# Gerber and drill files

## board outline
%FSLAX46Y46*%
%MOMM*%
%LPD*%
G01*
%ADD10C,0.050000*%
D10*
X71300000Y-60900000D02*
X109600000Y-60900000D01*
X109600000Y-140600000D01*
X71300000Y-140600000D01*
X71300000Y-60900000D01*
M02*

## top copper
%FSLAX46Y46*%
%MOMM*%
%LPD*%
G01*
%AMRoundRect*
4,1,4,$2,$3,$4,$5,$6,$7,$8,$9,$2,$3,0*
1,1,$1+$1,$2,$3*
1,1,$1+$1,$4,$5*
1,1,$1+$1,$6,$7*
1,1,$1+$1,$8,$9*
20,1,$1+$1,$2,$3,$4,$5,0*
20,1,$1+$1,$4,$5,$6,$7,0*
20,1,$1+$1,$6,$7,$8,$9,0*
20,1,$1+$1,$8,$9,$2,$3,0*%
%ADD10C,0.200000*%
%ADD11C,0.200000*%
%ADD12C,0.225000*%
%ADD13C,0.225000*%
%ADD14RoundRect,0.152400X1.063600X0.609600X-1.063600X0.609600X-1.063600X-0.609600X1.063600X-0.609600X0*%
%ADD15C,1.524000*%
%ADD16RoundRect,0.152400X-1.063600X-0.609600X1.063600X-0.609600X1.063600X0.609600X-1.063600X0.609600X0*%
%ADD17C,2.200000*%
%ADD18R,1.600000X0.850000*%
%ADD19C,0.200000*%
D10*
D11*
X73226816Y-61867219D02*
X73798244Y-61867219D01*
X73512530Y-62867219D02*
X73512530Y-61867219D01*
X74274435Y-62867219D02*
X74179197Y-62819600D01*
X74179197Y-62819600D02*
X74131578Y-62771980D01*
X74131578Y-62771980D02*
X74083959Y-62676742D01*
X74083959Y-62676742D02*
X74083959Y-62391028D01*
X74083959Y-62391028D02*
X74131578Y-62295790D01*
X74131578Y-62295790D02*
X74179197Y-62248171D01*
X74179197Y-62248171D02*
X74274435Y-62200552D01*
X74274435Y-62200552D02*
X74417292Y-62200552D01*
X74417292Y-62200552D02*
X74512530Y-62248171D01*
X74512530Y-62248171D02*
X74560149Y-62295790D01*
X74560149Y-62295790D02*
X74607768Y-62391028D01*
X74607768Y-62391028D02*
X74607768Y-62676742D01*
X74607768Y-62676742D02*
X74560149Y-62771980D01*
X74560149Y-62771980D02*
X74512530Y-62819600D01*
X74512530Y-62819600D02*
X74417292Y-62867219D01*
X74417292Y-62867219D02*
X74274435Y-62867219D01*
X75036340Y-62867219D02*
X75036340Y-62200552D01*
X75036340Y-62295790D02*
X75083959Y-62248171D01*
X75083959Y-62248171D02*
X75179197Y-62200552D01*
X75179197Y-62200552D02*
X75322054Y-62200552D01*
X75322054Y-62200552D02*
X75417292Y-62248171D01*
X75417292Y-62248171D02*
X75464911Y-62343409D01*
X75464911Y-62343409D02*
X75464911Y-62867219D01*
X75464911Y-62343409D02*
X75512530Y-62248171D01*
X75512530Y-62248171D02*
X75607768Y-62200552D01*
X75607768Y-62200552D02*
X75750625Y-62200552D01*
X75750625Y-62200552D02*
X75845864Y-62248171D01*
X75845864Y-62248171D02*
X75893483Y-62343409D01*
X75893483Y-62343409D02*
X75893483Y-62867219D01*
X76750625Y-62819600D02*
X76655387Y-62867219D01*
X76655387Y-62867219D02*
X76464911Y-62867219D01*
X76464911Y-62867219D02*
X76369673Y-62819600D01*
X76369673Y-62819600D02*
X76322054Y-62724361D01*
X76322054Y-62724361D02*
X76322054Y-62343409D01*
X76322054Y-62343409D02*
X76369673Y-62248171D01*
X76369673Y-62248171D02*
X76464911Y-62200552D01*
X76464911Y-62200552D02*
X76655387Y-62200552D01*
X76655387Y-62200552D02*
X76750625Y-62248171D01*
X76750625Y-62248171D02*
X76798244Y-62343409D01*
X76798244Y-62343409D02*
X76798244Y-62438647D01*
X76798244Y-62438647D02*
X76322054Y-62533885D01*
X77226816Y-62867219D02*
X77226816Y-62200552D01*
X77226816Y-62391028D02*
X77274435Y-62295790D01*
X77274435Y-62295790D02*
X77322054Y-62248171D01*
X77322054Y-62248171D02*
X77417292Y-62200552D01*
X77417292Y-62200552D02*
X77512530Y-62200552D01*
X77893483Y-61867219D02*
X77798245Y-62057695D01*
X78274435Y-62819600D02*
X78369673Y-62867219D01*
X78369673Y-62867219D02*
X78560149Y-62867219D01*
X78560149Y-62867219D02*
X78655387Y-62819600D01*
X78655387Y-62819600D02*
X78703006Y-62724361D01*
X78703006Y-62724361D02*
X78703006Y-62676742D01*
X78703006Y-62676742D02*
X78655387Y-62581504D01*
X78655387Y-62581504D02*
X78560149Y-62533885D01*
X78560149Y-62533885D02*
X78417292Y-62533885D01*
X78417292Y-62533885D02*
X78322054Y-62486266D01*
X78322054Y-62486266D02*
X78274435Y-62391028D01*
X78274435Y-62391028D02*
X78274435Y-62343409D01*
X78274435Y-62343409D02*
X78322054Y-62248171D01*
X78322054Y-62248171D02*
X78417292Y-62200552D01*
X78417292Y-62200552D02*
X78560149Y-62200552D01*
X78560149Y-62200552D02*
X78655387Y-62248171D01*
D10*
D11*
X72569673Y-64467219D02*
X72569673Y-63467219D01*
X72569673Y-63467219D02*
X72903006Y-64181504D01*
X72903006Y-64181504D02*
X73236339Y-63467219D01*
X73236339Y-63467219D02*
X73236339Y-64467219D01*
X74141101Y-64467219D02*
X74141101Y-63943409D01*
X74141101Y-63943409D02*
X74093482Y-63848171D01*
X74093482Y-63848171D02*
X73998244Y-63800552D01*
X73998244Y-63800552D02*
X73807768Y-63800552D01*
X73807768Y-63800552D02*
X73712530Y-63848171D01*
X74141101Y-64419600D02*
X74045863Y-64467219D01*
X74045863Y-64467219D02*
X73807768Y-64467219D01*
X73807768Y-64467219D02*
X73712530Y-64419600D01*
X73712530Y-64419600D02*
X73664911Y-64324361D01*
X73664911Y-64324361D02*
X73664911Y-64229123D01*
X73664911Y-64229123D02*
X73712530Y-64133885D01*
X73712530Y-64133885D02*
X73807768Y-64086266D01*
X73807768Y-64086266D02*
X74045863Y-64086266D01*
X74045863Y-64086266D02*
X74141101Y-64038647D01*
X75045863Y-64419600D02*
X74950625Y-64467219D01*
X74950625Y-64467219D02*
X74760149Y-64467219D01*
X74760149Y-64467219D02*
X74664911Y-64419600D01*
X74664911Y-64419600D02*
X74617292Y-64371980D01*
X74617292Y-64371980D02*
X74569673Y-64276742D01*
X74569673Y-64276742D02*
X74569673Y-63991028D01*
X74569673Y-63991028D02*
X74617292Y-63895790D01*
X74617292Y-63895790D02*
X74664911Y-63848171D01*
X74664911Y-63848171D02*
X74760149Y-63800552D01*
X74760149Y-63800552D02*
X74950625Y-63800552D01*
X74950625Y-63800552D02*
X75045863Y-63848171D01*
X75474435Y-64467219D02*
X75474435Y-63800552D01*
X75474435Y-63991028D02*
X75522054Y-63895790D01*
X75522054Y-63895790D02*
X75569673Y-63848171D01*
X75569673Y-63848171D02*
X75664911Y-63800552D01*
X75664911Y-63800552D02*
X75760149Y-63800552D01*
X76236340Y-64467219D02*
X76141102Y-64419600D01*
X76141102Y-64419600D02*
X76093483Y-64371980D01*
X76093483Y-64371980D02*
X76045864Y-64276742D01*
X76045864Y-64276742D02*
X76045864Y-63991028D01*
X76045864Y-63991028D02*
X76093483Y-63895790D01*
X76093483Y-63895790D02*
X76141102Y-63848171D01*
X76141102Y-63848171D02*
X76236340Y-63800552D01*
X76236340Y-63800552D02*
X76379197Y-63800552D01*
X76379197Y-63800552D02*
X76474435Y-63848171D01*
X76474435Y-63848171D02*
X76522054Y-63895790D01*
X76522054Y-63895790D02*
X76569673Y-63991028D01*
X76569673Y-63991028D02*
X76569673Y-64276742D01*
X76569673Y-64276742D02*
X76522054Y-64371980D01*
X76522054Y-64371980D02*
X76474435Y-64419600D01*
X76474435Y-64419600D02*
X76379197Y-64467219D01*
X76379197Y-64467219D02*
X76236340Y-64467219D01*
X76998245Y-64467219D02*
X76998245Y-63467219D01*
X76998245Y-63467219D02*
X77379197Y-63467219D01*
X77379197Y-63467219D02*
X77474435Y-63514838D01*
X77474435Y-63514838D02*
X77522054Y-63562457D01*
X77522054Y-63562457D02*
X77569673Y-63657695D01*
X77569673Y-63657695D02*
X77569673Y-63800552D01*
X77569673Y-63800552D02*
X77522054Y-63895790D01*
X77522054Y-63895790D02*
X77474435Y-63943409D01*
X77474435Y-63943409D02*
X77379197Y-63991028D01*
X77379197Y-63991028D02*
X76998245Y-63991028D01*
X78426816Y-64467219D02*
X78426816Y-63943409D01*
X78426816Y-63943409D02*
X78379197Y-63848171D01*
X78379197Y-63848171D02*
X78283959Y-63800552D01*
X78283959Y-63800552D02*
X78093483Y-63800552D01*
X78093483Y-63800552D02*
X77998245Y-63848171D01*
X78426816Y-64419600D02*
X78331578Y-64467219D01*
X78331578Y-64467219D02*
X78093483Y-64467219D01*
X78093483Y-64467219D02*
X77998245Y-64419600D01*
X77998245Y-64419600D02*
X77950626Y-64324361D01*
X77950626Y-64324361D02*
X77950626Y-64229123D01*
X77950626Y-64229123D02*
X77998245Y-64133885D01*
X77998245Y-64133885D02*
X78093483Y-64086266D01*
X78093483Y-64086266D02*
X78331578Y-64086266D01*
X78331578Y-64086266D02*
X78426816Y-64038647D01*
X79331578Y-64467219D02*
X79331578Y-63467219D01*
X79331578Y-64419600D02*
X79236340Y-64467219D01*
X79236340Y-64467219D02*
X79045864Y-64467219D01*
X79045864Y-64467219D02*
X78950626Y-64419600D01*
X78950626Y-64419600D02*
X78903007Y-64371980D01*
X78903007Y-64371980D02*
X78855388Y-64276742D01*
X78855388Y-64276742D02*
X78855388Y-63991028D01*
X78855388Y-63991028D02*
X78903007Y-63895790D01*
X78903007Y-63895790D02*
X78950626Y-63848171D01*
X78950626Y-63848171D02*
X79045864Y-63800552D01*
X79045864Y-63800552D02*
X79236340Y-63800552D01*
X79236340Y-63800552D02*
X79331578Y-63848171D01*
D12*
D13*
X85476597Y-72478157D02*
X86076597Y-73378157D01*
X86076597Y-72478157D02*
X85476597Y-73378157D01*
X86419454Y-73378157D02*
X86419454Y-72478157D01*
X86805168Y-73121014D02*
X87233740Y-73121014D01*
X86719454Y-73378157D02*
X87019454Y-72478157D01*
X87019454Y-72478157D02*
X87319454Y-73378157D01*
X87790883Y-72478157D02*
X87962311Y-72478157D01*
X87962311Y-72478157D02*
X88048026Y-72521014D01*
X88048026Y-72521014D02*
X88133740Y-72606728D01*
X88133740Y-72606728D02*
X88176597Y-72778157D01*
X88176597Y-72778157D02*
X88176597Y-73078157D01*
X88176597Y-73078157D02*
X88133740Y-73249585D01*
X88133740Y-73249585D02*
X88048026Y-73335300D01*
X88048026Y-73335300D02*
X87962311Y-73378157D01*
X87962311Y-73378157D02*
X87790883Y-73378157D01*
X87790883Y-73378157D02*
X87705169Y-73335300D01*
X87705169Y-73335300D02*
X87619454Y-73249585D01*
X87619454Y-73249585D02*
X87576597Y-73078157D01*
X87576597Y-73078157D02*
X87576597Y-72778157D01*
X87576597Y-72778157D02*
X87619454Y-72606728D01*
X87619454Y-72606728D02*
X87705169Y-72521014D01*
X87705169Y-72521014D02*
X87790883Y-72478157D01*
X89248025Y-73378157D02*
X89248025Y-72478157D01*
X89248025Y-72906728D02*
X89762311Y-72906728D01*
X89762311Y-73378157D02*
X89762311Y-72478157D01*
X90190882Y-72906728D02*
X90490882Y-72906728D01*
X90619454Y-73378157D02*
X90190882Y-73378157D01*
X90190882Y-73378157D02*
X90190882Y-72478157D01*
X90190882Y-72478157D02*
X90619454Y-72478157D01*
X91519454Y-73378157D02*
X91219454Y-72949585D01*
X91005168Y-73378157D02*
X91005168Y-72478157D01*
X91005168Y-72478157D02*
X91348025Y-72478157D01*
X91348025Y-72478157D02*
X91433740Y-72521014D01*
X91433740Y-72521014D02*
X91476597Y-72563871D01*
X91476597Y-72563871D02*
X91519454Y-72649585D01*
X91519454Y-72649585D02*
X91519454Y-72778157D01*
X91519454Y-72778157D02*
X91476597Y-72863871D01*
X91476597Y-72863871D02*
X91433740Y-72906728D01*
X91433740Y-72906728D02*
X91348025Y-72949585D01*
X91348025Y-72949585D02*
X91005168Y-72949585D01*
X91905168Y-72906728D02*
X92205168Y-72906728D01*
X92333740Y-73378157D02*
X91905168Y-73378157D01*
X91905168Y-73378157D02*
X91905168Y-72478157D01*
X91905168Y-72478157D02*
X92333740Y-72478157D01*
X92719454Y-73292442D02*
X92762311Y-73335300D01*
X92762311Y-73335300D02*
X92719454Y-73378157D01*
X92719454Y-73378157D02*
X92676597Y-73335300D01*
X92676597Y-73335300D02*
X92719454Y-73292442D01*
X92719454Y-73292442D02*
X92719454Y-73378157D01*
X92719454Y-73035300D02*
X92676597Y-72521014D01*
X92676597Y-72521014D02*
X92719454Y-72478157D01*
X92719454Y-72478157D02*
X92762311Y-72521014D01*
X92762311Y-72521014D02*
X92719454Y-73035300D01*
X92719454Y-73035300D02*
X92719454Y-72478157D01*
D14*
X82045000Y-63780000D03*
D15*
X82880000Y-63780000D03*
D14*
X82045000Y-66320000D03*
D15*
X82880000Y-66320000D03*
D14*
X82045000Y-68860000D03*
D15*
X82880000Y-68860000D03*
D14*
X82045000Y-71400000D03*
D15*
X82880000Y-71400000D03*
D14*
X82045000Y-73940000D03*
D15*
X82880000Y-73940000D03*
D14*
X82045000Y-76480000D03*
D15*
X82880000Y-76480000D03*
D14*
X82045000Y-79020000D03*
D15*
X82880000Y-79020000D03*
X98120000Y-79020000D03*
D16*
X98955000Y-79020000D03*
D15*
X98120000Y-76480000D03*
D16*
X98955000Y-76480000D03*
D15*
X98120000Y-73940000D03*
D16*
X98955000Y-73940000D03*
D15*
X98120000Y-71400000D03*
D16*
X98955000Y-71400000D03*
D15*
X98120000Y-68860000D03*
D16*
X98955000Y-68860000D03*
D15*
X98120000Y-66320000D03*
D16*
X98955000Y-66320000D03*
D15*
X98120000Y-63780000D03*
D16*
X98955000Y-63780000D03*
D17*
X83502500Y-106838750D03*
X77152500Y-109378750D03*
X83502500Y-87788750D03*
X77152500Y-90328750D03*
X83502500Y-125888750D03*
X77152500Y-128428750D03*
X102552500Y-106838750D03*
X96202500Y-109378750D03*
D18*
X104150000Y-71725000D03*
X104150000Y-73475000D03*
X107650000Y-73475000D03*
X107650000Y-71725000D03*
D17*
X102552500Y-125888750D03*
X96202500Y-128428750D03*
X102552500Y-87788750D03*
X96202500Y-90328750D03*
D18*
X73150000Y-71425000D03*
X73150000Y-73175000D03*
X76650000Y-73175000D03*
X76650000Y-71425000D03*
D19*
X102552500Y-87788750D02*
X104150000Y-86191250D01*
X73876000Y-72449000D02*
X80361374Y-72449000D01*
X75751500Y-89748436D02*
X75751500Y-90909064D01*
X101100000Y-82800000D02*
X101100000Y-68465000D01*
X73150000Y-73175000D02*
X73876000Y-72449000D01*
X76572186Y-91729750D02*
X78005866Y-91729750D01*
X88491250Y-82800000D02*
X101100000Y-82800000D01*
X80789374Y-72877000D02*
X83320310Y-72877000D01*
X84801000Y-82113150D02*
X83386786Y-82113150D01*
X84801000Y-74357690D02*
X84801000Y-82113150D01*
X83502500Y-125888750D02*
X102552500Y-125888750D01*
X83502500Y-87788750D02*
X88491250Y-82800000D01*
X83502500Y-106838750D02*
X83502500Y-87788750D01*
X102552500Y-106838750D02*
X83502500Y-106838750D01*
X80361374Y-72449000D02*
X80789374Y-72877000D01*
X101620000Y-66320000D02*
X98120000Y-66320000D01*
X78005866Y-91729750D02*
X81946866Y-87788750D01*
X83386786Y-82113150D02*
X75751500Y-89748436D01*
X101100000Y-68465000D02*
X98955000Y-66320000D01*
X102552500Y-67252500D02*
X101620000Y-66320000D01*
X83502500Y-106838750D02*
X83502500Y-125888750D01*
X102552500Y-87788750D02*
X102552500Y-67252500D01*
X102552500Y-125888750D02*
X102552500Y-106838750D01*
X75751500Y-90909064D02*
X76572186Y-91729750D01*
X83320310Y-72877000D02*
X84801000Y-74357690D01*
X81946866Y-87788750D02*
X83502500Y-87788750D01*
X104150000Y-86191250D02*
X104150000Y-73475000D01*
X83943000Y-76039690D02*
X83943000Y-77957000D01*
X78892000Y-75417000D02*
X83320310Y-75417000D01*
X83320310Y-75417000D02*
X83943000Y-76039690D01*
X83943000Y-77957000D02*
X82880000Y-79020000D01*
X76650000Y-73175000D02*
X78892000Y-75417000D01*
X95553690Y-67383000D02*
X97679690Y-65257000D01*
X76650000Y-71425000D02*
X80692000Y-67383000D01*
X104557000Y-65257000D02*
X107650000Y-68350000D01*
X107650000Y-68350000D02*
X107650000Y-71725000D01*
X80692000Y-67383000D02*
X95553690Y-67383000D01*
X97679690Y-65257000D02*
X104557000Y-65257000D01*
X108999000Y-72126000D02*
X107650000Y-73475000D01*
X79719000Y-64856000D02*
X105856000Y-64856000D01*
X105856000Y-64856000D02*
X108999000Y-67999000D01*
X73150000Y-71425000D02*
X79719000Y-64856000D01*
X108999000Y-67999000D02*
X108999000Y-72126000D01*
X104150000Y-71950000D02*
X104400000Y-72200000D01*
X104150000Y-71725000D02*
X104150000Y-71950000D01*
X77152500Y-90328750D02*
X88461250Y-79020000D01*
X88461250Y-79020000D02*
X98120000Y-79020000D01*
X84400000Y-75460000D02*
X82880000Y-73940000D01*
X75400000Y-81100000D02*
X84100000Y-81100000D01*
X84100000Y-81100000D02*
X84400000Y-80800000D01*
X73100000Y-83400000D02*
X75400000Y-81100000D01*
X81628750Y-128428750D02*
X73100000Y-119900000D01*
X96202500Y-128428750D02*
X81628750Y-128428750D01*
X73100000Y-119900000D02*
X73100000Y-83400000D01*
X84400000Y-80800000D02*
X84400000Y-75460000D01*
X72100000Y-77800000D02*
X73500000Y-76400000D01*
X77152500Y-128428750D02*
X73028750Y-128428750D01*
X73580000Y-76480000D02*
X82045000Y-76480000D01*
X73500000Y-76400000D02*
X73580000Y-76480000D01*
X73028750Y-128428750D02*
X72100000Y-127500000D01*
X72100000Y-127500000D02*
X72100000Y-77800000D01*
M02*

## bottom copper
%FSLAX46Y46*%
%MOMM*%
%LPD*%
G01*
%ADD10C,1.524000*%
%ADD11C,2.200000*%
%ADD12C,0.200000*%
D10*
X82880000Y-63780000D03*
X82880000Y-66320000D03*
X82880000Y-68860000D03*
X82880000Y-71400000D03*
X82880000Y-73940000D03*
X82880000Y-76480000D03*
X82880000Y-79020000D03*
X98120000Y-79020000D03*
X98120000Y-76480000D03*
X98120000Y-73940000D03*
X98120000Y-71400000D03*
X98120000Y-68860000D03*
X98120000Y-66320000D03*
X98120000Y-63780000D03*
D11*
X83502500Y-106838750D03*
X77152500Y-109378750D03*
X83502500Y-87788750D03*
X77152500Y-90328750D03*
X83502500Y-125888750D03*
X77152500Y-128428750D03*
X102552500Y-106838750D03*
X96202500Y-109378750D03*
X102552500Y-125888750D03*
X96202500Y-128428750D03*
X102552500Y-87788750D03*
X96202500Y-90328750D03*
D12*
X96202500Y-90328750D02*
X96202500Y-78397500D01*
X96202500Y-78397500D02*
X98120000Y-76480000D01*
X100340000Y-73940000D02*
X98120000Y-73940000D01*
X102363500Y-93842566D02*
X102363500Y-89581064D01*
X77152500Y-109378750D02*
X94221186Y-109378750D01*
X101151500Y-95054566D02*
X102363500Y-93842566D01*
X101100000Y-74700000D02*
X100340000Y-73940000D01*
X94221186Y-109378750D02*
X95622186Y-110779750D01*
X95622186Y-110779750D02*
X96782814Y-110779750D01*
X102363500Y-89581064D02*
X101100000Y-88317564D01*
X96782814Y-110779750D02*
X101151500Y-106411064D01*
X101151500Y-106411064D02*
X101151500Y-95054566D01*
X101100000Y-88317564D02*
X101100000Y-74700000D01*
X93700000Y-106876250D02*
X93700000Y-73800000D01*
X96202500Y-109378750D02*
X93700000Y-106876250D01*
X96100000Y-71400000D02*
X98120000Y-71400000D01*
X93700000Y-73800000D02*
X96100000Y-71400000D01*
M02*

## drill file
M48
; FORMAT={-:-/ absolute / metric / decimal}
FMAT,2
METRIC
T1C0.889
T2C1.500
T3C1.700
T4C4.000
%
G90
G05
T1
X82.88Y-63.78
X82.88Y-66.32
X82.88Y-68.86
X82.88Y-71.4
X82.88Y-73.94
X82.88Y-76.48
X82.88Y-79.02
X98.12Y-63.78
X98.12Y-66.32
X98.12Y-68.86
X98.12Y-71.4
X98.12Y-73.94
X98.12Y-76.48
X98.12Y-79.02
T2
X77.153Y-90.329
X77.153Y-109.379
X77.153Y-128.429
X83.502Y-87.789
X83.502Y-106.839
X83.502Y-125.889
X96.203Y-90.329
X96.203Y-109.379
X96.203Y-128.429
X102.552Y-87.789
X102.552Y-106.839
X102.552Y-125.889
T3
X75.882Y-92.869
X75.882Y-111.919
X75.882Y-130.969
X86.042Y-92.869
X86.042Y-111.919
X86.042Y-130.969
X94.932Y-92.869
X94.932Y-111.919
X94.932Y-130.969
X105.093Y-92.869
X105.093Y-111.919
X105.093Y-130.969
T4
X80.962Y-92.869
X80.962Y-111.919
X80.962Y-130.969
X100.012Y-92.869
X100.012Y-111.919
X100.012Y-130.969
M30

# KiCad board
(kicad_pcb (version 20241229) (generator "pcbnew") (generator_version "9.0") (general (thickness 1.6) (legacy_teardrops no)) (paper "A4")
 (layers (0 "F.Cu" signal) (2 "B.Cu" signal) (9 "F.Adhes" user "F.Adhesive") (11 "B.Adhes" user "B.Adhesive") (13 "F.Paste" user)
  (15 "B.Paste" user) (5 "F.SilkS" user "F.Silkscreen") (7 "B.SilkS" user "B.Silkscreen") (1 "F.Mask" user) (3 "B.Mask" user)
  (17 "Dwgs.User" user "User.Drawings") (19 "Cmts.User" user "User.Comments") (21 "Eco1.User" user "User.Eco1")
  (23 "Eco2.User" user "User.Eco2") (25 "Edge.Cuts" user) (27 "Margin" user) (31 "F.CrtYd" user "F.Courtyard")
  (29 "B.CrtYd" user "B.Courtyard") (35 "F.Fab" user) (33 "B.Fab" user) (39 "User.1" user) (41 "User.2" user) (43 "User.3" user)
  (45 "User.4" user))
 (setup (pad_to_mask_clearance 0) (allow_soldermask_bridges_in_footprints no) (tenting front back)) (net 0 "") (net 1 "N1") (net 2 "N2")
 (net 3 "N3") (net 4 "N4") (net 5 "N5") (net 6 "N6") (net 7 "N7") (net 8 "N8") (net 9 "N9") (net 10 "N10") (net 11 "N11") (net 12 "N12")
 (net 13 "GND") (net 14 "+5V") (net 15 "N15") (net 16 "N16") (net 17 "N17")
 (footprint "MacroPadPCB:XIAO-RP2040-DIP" (layer "F.Cu") (at 90.5 71.4)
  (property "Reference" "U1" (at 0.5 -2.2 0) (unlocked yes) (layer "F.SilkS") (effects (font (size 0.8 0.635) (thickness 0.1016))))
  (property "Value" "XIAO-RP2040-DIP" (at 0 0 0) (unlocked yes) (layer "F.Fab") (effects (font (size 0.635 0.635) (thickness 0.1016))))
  (pad "1" smd roundrect (at -8.455 -7.62 180) (size 2.432 1.524) (layers "F.Cu" "F.Mask") (roundrect_rratio 0.1) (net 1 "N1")
   (thermal_bridge_angle 45))
  (pad "1" thru_hole circle (at -7.62 -7.62 180) (size 1.524 1.524) (drill 0.889) (layers "*.Cu" "*.Mask") (remove_unused_layers no)
   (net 1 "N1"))
  (pad "2" smd roundrect (at -8.455 -5.08 180) (size 2.432 1.524) (layers "F.Cu" "F.Mask") (roundrect_rratio 0.1) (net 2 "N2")
   (thermal_bridge_angle 45))
  (pad "2" thru_hole circle (at -7.62 -5.08 180) (size 1.524 1.524) (drill 0.889) (layers "*.Cu" "*.Mask") (remove_unused_layers no)
   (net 2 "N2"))
  (pad "3" smd roundrect (at -8.455 -2.54 180) (size 2.432 1.524) (layers "F.Cu" "F.Mask") (roundrect_rratio 0.1) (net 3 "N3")
   (thermal_bridge_angle 45))
  (pad "3" thru_hole circle (at -7.62 -2.54 180) (size 1.524 1.524) (drill 0.889) (layers "*.Cu" "*.Mask") (remove_unused_layers no)
   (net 3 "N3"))
  (pad "4" smd roundrect (at -8.455 0 180) (size 2.432 1.524) (layers "F.Cu" "F.Mask") (roundrect_rratio 0.1) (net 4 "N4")
   (thermal_bridge_angle 45))
  (pad "4" thru_hole circle (at -7.62 0 180) (size 1.524 1.524) (drill 0.889) (layers "*.Cu" "*.Mask") (remove_unused_layers no)
   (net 4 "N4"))
  (pad "5" smd roundrect (at -8.455 2.54 180) (size 2.432 1.524) (layers "F.Cu" "F.Mask") (roundrect_rratio 0.1) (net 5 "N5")
   (thermal_bridge_angle 45))
  (pad "5" thru_hole circle (at -7.62 2.54 180) (size 1.524 1.524) (drill 0.889) (layers "*.Cu" "*.Mask") (remove_unused_layers no)
   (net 5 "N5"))
  (pad "6" smd roundrect (at -8.455 5.08 180) (size 2.432 1.524) (layers "F.Cu" "F.Mask") (roundrect_rratio 0.1) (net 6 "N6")
   (thermal_bridge_angle 45))
  (pad "6" thru_hole circle (at -7.62 5.08 180) (size 1.524 1.524) (drill 0.889) (layers "*.Cu" "*.Mask") (remove_unused_layers no)
   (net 6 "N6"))
  (pad "7" smd roundrect (at -8.455 7.62 180) (size 2.432 1.524) (layers "F.Cu" "F.Mask") (roundrect_rratio 0.1) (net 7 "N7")
   (thermal_bridge_angle 45))
  (pad "7" thru_hole circle (at -7.62 7.62 180) (size 1.524 1.524) (drill 0.889) (layers "*.Cu" "*.Mask") (remove_unused_layers no)
   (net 7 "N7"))
  (pad "8" thru_hole circle (at 7.62 7.62) (size 1.524 1.524) (drill 0.889) (layers "*.Cu" "*.Mask") (remove_unused_layers no) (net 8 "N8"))
  (pad "8" smd roundrect (at 8.455 7.62) (size 2.432 1.524) (layers "F.Cu" "F.Mask") (roundrect_rratio 0.1) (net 8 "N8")
   (thermal_bridge_angle 45))
  (pad "9" thru_hole circle (at 7.62 5.08) (size 1.524 1.524) (drill 0.889) (layers "*.Cu" "*.Mask") (remove_unused_layers no) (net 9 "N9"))
  (pad "9" smd roundrect (at 8.455 5.08) (size 2.432 1.524) (layers "F.Cu" "F.Mask") (roundrect_rratio 0.1) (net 9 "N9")
   (thermal_bridge_angle 45))
  (pad "10" thru_hole circle (at 7.62 2.54) (size 1.524 1.524) (drill 0.889) (layers "*.Cu" "*.Mask") (remove_unused_layers no)
   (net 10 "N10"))
  (pad "10" smd roundrect (at 8.455 2.54) (size 2.432 1.524) (layers "F.Cu" "F.Mask") (roundrect_rratio 0.1) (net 10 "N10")
   (thermal_bridge_angle 45))
  (pad "11" thru_hole circle (at 7.62 0) (size 1.524 1.524) (drill 0.889) (layers "*.Cu" "*.Mask") (remove_unused_layers no) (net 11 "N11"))
  (pad "11" smd roundrect (at 8.455 0) (size 2.432 1.524) (layers "F.Cu" "F.Mask") (roundrect_rratio 0.1) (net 11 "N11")
   (thermal_bridge_angle 45))
  (pad "12" thru_hole circle (at 7.62 -2.54) (size 1.524 1.524) (drill 0.889) (layers "*.Cu" "*.Mask") (remove_unused_layers no)
   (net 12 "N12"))
  (pad "12" smd roundrect (at 8.455 -2.54) (size 2.432 1.524) (layers "F.Cu" "F.Mask") (roundrect_rratio 0.1) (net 12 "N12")
   (thermal_bridge_angle 45))
  (pad "13" thru_hole circle (at 7.62 -5.08) (size 1.524 1.524) (drill 0.889) (layers "*.Cu" "*.Mask") (remove_unused_layers no)
   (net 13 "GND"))
  (pad "13" smd roundrect (at 8.455 -5.08) (size 2.432 1.524) (layers "F.Cu" "F.Mask") (roundrect_rratio 0.1) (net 13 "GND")
   (thermal_bridge_angle 45))
  (pad "14" thru_hole circle (at 7.62 -7.62) (size 1.524 1.524) (drill 0.889) (layers "*.Cu" "*.Mask") (remove_unused_layers no)
   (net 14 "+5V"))
  (pad "14" smd roundrect (at 8.455 -7.62) (size 2.432 1.524) (layers "F.Cu" "F.Mask") (roundrect_rratio 0.1) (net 14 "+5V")
   (thermal_bridge_angle 45)))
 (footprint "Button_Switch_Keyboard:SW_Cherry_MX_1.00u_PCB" (layer "F.Cu") (at 83.5025 106.83875)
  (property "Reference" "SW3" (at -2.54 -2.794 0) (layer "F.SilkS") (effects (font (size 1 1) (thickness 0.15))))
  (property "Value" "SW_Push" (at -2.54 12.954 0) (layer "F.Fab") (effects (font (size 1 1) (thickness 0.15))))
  (pad "" np_thru_hole circle (at -7.62 5.08) (size 1.7 1.7) (drill 1.7) (layers "*.Cu" "*.Mask"))
  (pad "" np_thru_hole circle (at -2.54 5.08) (size 4 4) (drill 4) (layers "*.Cu" "*.Mask"))
  (pad "" np_thru_hole circle (at 2.54 5.08) (size 1.7 1.7) (drill 1.7) (layers "*.Cu" "*.Mask"))
  (pad "1" thru_hole circle (at 0 0) (size 2.2 2.2) (drill 1.5) (layers "*.Cu" "*.Mask") (remove_unused_layers no) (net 13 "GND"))
  (pad "2" thru_hole circle (at -6.35 2.54) (size 2.2 2.2) (drill 1.5) (layers "*.Cu" "*.Mask") (remove_unused_layers no) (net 10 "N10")))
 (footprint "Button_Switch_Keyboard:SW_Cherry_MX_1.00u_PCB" (layer "F.Cu") (at 83.5025 87.78875)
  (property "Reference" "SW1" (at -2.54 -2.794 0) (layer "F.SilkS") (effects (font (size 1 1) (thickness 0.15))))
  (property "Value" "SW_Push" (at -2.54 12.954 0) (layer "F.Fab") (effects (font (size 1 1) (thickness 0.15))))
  (pad "" np_thru_hole circle (at -7.62 5.08) (size 1.7 1.7) (drill 1.7) (layers "*.Cu" "*.Mask"))
  (pad "" np_thru_hole circle (at -2.54 5.08) (size 4 4) (drill 4) (layers "*.Cu" "*.Mask"))
  (pad "" np_thru_hole circle (at 2.54 5.08) (size 1.7 1.7) (drill 1.7) (layers "*.Cu" "*.Mask"))
  (pad "1" thru_hole circle (at 0 0) (size 2.2 2.2) (drill 1.5) (layers "*.Cu" "*.Mask") (remove_unused_layers no) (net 13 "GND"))
  (pad "2" thru_hole circle (at -6.35 2.54) (size 2.2 2.2) (drill 1.5) (layers "*.Cu" "*.Mask") (remove_unused_layers no) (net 8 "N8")))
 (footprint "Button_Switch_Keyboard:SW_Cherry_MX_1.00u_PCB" (layer "F.Cu") (at 83.5025 125.88875)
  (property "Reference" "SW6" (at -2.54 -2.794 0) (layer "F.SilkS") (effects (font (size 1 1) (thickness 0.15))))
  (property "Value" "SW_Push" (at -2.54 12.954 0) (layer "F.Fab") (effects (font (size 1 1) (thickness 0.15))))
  (pad "" np_thru_hole circle (at -7.62 5.08) (size 1.7 1.7) (drill 1.7) (layers "*.Cu" "*.Mask"))
  (pad "" np_thru_hole circle (at -2.54 5.08) (size 4 4) (drill 4) (layers "*.Cu" "*.Mask"))
  (pad "" np_thru_hole circle (at 2.54 5.08) (size 1.7 1.7) (drill 1.7) (layers "*.Cu" "*.Mask"))
  (pad "1" thru_hole circle (at 0 0) (size 2.2 2.2) (drill 1.5) (layers "*.Cu" "*.Mask") (remove_unused_layers no) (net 13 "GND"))
  (pad "2" thru_hole circle (at -6.35 2.54) (size 2.2 2.2) (drill 1.5) (layers "*.Cu" "*.Mask") (remove_unused_layers no) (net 6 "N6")))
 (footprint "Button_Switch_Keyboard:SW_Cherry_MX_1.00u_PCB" (layer "F.Cu") (at 102.5525 106.83875)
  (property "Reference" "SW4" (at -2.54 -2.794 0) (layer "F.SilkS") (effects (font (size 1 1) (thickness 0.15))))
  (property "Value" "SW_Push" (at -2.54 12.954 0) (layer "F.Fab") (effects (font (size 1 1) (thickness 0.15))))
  (pad "" np_thru_hole circle (at -7.62 5.08) (size 1.7 1.7) (drill 1.7) (layers "*.Cu" "*.Mask"))
  (pad "" np_thru_hole circle (at -2.54 5.08) (size 4 4) (drill 4) (layers "*.Cu" "*.Mask"))
  (pad "" np_thru_hole circle (at 2.54 5.08) (size 1.7 1.7) (drill 1.7) (layers "*.Cu" "*.Mask"))
  (pad "1" thru_hole circle (at 0 0) (size 2.2 2.2) (drill 1.5) (layers "*.Cu" "*.Mask") (remove_unused_layers no) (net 13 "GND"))
  (pad "2" thru_hole circle (at -6.35 2.54) (size 2.2 2.2) (drill 1.5) (layers "*.Cu" "*.Mask") (remove_unused_layers no) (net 11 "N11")))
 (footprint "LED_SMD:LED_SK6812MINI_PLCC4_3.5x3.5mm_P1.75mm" (layer "F.Cu") (at 105.9 72.6)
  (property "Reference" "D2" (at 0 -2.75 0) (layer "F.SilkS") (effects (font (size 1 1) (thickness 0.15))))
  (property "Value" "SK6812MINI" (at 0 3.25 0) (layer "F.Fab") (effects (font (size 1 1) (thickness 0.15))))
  (pad "1" smd rect (at -1.75 -0.875) (size 1.6 0.85) (layers "F.Cu" "F.Mask" "F.Paste") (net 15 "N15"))
  (pad "2" smd rect (at -1.75 0.875) (size 1.6 0.85) (layers "F.Cu" "F.Mask" "F.Paste") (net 13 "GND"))
  (pad "3" smd rect (at 1.75 0.875) (size 1.6 0.85) (layers "F.Cu" "F.Mask" "F.Paste") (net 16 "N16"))
  (pad "4" smd rect (at 1.75 -0.875) (size 1.6 0.85) (layers "F.Cu" "F.Mask" "F.Paste") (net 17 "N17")))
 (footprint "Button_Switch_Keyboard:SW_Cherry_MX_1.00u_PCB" (layer "F.Cu") (at 102.5525 125.88875)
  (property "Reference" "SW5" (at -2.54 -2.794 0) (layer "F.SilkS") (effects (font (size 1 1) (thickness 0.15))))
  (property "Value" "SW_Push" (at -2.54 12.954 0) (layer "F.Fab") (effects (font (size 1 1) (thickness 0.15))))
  (pad "" np_thru_hole circle (at -7.62 5.08) (size 1.7 1.7) (drill 1.7) (layers "*.Cu" "*.Mask"))
  (pad "" np_thru_hole circle (at -2.54 5.08) (size 4 4) (drill 4) (layers "*.Cu" "*.Mask"))
  (pad "" np_thru_hole circle (at 2.54 5.08) (size 1.7 1.7) (drill 1.7) (layers "*.Cu" "*.Mask"))
  (pad "1" thru_hole circle (at 0 0) (size 2.2 2.2) (drill 1.5) (layers "*.Cu" "*.Mask") (remove_unused_layers no) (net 13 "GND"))
  (pad "2" thru_hole circle (at -6.35 2.54) (size 2.2 2.2) (drill 1.5) (layers "*.Cu" "*.Mask") (remove_unused_layers no) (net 5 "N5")))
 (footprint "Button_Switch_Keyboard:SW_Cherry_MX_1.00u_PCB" (layer "F.Cu") (at 102.5525 87.78875)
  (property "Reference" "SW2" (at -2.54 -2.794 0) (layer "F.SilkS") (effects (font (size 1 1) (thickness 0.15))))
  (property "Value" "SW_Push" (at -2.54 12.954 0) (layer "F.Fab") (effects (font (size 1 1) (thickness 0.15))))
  (pad "" np_thru_hole circle (at -7.62 5.08) (size 1.7 1.7) (drill 1.7) (layers "*.Cu" "*.Mask"))
  (pad "" np_thru_hole circle (at -2.54 5.08) (size 4 4) (drill 4) (layers "*.Cu" "*.Mask"))
  (pad "" np_thru_hole circle (at 2.54 5.08) (size 1.7 1.7) (drill 1.7) (layers "*.Cu" "*.Mask"))
  (pad "1" thru_hole circle (at 0 0) (size 2.2 2.2) (drill 1.5) (layers "*.Cu" "*.Mask") (remove_unused_layers no) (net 13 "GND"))
  (pad "2" thru_hole circle (at -6.35 2.54) (size 2.2 2.2) (drill 1.5) (layers "*.Cu" "*.Mask") (remove_unused_layers no) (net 9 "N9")))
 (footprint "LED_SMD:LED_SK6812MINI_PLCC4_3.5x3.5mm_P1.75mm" (layer "F.Cu") (at 74.9 72.3)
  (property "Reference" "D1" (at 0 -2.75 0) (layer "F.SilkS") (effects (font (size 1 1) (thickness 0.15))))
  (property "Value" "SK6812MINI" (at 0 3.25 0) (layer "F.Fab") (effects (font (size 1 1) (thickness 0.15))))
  (pad "1" smd rect (at -1.75 -0.875) (size 1.6 0.85) (layers "F.Cu" "F.Mask" "F.Paste") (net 16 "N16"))
  (pad "2" smd rect (at -1.75 0.875) (size 1.6 0.85) (layers "F.Cu" "F.Mask" "F.Paste") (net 13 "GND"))
  (pad "3" smd rect (at 1.75 0.875) (size 1.6 0.85) (layers "F.Cu" "F.Mask" "F.Paste") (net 7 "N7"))
  (pad "4" smd rect (at 1.75 -0.875) (size 1.6 0.85) (layers "F.Cu" "F.Mask" "F.Paste") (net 17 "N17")))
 (gr_rect (start 71.3 60.9) (end 109.6 140.6) (stroke (width 0.05) (type default)) (fill no) (layer "Edge.Cuts"))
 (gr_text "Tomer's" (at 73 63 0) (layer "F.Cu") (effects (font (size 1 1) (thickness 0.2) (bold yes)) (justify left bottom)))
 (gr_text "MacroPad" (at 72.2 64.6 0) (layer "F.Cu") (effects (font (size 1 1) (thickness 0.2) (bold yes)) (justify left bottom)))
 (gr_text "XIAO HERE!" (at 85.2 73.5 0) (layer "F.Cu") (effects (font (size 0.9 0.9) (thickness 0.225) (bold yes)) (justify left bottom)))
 (segment (start 102.5525 87.78875) (end 104.15 86.19125) (width 0.2) (layer "F.Cu") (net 13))
 (segment (start 73.876 72.449) (end 80.361374 72.449) (width 0.2) (layer "F.Cu") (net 13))
 (segment (start 75.7515 89.748436) (end 75.7515 90.909064) (width 0.2) (layer "F.Cu") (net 13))
 (segment (start 101.1 82.8) (end 101.1 68.465) (width 0.2) (layer "F.Cu") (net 13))
 (segment (start 73.15 73.175) (end 73.876 72.449) (width 0.2) (layer "F.Cu") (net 13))
 (segment (start 76.572186 91.72975) (end 78.005866 91.72975) (width 0.2) (layer "F.Cu") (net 13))
 (segment (start 88.49125 82.8) (end 101.1 82.8) (width 0.2) (layer "F.Cu") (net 13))
 (segment (start 80.789374 72.877) (end 83.32031 72.877) (width 0.2) (layer "F.Cu") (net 13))
 (segment (start 84.801 82.11315) (end 83.386786 82.11315) (width 0.2) (layer "F.Cu") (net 13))
 (segment (start 84.801 74.35769) (end 84.801 82.11315) (width 0.2) (layer "F.Cu") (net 13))
 (segment (start 83.5025 125.88875) (end 102.5525 125.88875) (width 0.2) (layer "F.Cu") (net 13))
 (segment (start 83.5025 87.78875) (end 88.49125 82.8) (width 0.2) (layer "F.Cu") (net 13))
 (segment (start 83.5025 106.83875) (end 83.5025 87.78875) (width 0.2) (layer "F.Cu") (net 13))
 (segment (start 102.5525 106.83875) (end 83.5025 106.83875) (width 0.2) (layer "F.Cu") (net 13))
 (segment (start 80.361374 72.449) (end 80.789374 72.877) (width 0.2) (layer "F.Cu") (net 13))
 (segment (start 101.62 66.32) (end 98.12 66.32) (width 0.2) (layer "F.Cu") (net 13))
 (segment (start 78.005866 91.72975) (end 81.946866 87.78875) (width 0.2) (layer "F.Cu") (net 13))
 (segment (start 83.386786 82.11315) (end 75.7515 89.748436) (width 0.2) (layer "F.Cu") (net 13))
 (segment (start 101.1 68.465) (end 98.955 66.32) (width 0.2) (layer "F.Cu") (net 13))
 (segment (start 102.5525 67.2525) (end 101.62 66.32) (width 0.2) (layer "F.Cu") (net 13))
 (segment (start 83.5025 106.83875) (end 83.5025 125.88875) (width 0.2) (layer "F.Cu") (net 13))
 (segment (start 102.5525 87.78875) (end 102.5525 67.2525) (width 0.2) (layer "F.Cu") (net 13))
 (segment (start 102.5525 125.88875) (end 102.5525 106.83875) (width 0.2) (layer "F.Cu") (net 13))
 (segment (start 75.7515 90.909064) (end 76.572186 91.72975) (width 0.2) (layer "F.Cu") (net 13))
 (segment (start 83.32031 72.877) (end 84.801 74.35769) (width 0.2) (layer "F.Cu") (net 13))
 (segment (start 81.946866 87.78875) (end 83.5025 87.78875) (width 0.2) (layer "F.Cu") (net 13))
 (segment (start 104.15 86.19125) (end 104.15 73.475) (width 0.2) (layer "F.Cu") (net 13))
 (segment (start 83.943 76.03969) (end 83.943 77.957) (width 0.2) (layer "F.Cu") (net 7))
 (segment (start 78.892 75.417) (end 83.32031 75.417) (width 0.2) (layer "F.Cu") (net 7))
 (segment (start 83.32031 75.417) (end 83.943 76.03969) (width 0.2) (layer "F.Cu") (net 7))
 (segment (start 83.943 77.957) (end 82.88 79.02) (width 0.2) (layer "F.Cu") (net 7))
 (segment (start 76.65 73.175) (end 78.892 75.417) (width 0.2) (layer "F.Cu") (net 7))
 (segment (start 95.55369 67.383) (end 97.67969 65.257) (width 0.2) (layer "F.Cu") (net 17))
 (segment (start 76.65 71.425) (end 80.692 67.383) (width 0.2) (layer "F.Cu") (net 17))
 (segment (start 104.557 65.257) (end 107.65 68.35) (width 0.2) (layer "F.Cu") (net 17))
 (segment (start 107.65 68.35) (end 107.65 71.725) (width 0.2) (layer "F.Cu") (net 17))
 (segment (start 80.692 67.383) (end 95.55369 67.383) (width 0.2) (layer "F.Cu") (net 17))
 (segment (start 97.67969 65.257) (end 104.557 65.257) (width 0.2) (layer "F.Cu") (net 17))
 (segment (start 108.999 72.126) (end 107.65 73.475) (width 0.2) (layer "F.Cu") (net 16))
 (segment (start 79.719 64.856) (end 105.856 64.856) (width 0.2) (layer "F.Cu") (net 16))
 (segment (start 105.856 64.856) (end 108.999 67.999) (width 0.2) (layer "F.Cu") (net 16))
 (segment (start 73.15 71.425) (end 79.719 64.856) (width 0.2) (layer "F.Cu") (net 16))
 (segment (start 108.999 67.999) (end 108.999 72.126) (width 0.2) (layer "F.Cu") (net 16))
 (segment (start 104.15 71.95) (end 104.4 72.2) (width 0.2) (layer "F.Cu") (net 15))
 (segment (start 104.15 71.725) (end 104.15 71.95) (width 0.2) (layer "F.Cu") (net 15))
 (segment (start 77.1525 90.32875) (end 88.46125 79.02) (width 0.2) (layer "F.Cu") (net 8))
 (segment (start 88.46125 79.02) (end 98.12 79.02) (width 0.2) (layer "F.Cu") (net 8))
 (segment (start 96.2025 90.32875) (end 96.2025 78.3975) (width 0.2) (layer "B.Cu") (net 9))
 (segment (start 96.2025 78.3975) (end 98.12 76.48) (width 0.2) (layer "B.Cu") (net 9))
 (segment (start 100.34 73.94) (end 98.12 73.94) (width 0.2) (layer "B.Cu") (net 10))
 (segment (start 102.3635 93.842566) (end 102.3635 89.581064) (width 0.2) (layer "B.Cu") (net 10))
 (segment (start 77.1525 109.37875) (end 94.221186 109.37875) (width 0.2) (layer "B.Cu") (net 10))
 (segment (start 101.1515 95.054566) (end 102.3635 93.842566) (width 0.2) (layer "B.Cu") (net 10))
 (segment (start 101.1 74.7) (end 100.34 73.94) (width 0.2) (layer "B.Cu") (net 10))
 (segment (start 94.221186 109.37875) (end 95.622186 110.77975) (width 0.2) (layer "B.Cu") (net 10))
 (segment (start 95.622186 110.77975) (end 96.782814 110.77975) (width 0.2) (layer "B.Cu") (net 10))
 (segment (start 102.3635 89.581064) (end 101.1 88.317564) (width 0.2) (layer "B.Cu") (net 10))
 (segment (start 96.782814 110.77975) (end 101.1515 106.411064) (width 0.2) (layer "B.Cu") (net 10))
 (segment (start 101.1515 106.411064) (end 101.1515 95.054566) (width 0.2) (layer "B.Cu") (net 10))
 (segment (start 101.1 88.317564) (end 101.1 74.7) (width 0.2) (layer "B.Cu") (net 10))
 (segment (start 93.7 106.87625) (end 93.7 73.8) (width 0.2) (layer "B.Cu") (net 11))
 (segment (start 96.2025 109.37875) (end 93.7 106.87625) (width 0.2) (layer "B.Cu") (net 11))
 (segment (start 96.1 71.4) (end 98.12 71.4) (width 0.2) (layer "B.Cu") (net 11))
 (segment (start 93.7 73.8) (end 96.1 71.4) (width 0.2) (layer "B.Cu") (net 11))
 (segment (start 84.4 75.46) (end 82.88 73.94) (width 0.2) (layer "F.Cu") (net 5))
 (segment (start 75.4 81.1) (end 84.1 81.1) (width 0.2) (layer "F.Cu") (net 5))
 (segment (start 84.1 81.1) (end 84.4 80.8) (width 0.2) (layer "F.Cu") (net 5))
 (segment (start 73.1 83.4) (end 75.4 81.1) (width 0.2) (layer "F.Cu") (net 5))
 (segment (start 81.62875 128.42875) (end 73.1 119.9) (width 0.2) (layer "F.Cu") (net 5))
 (segment (start 96.2025 128.42875) (end 81.62875 128.42875) (width 0.2) (layer "F.Cu") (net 5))
 (segment (start 73.1 119.9) (end 73.1 83.4) (width 0.2) (layer "F.Cu") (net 5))
 (segment (start 84.4 80.8) (end 84.4 75.46) (width 0.2) (layer "F.Cu") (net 5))
 (segment (start 72.1 77.8) (end 73.5 76.4) (width 0.2) (layer "F.Cu") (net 6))
 (segment (start 77.1525 128.42875) (end 73.02875 128.42875) (width 0.2) (layer "F.Cu") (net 6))
 (segment (start 73.58 76.48) (end 82.045 76.48) (width 0.2) (layer "F.Cu") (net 6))
 (segment (start 73.5 76.4) (end 73.58 76.48) (width 0.2) (layer "F.Cu") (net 6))
 (segment (start 73.02875 128.42875) (end 72.1 127.5) (width 0.2) (layer "F.Cu") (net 6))
 (segment (start 72.1 127.5) (end 72.1 77.8) (width 0.2) (layer "F.Cu") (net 6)))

